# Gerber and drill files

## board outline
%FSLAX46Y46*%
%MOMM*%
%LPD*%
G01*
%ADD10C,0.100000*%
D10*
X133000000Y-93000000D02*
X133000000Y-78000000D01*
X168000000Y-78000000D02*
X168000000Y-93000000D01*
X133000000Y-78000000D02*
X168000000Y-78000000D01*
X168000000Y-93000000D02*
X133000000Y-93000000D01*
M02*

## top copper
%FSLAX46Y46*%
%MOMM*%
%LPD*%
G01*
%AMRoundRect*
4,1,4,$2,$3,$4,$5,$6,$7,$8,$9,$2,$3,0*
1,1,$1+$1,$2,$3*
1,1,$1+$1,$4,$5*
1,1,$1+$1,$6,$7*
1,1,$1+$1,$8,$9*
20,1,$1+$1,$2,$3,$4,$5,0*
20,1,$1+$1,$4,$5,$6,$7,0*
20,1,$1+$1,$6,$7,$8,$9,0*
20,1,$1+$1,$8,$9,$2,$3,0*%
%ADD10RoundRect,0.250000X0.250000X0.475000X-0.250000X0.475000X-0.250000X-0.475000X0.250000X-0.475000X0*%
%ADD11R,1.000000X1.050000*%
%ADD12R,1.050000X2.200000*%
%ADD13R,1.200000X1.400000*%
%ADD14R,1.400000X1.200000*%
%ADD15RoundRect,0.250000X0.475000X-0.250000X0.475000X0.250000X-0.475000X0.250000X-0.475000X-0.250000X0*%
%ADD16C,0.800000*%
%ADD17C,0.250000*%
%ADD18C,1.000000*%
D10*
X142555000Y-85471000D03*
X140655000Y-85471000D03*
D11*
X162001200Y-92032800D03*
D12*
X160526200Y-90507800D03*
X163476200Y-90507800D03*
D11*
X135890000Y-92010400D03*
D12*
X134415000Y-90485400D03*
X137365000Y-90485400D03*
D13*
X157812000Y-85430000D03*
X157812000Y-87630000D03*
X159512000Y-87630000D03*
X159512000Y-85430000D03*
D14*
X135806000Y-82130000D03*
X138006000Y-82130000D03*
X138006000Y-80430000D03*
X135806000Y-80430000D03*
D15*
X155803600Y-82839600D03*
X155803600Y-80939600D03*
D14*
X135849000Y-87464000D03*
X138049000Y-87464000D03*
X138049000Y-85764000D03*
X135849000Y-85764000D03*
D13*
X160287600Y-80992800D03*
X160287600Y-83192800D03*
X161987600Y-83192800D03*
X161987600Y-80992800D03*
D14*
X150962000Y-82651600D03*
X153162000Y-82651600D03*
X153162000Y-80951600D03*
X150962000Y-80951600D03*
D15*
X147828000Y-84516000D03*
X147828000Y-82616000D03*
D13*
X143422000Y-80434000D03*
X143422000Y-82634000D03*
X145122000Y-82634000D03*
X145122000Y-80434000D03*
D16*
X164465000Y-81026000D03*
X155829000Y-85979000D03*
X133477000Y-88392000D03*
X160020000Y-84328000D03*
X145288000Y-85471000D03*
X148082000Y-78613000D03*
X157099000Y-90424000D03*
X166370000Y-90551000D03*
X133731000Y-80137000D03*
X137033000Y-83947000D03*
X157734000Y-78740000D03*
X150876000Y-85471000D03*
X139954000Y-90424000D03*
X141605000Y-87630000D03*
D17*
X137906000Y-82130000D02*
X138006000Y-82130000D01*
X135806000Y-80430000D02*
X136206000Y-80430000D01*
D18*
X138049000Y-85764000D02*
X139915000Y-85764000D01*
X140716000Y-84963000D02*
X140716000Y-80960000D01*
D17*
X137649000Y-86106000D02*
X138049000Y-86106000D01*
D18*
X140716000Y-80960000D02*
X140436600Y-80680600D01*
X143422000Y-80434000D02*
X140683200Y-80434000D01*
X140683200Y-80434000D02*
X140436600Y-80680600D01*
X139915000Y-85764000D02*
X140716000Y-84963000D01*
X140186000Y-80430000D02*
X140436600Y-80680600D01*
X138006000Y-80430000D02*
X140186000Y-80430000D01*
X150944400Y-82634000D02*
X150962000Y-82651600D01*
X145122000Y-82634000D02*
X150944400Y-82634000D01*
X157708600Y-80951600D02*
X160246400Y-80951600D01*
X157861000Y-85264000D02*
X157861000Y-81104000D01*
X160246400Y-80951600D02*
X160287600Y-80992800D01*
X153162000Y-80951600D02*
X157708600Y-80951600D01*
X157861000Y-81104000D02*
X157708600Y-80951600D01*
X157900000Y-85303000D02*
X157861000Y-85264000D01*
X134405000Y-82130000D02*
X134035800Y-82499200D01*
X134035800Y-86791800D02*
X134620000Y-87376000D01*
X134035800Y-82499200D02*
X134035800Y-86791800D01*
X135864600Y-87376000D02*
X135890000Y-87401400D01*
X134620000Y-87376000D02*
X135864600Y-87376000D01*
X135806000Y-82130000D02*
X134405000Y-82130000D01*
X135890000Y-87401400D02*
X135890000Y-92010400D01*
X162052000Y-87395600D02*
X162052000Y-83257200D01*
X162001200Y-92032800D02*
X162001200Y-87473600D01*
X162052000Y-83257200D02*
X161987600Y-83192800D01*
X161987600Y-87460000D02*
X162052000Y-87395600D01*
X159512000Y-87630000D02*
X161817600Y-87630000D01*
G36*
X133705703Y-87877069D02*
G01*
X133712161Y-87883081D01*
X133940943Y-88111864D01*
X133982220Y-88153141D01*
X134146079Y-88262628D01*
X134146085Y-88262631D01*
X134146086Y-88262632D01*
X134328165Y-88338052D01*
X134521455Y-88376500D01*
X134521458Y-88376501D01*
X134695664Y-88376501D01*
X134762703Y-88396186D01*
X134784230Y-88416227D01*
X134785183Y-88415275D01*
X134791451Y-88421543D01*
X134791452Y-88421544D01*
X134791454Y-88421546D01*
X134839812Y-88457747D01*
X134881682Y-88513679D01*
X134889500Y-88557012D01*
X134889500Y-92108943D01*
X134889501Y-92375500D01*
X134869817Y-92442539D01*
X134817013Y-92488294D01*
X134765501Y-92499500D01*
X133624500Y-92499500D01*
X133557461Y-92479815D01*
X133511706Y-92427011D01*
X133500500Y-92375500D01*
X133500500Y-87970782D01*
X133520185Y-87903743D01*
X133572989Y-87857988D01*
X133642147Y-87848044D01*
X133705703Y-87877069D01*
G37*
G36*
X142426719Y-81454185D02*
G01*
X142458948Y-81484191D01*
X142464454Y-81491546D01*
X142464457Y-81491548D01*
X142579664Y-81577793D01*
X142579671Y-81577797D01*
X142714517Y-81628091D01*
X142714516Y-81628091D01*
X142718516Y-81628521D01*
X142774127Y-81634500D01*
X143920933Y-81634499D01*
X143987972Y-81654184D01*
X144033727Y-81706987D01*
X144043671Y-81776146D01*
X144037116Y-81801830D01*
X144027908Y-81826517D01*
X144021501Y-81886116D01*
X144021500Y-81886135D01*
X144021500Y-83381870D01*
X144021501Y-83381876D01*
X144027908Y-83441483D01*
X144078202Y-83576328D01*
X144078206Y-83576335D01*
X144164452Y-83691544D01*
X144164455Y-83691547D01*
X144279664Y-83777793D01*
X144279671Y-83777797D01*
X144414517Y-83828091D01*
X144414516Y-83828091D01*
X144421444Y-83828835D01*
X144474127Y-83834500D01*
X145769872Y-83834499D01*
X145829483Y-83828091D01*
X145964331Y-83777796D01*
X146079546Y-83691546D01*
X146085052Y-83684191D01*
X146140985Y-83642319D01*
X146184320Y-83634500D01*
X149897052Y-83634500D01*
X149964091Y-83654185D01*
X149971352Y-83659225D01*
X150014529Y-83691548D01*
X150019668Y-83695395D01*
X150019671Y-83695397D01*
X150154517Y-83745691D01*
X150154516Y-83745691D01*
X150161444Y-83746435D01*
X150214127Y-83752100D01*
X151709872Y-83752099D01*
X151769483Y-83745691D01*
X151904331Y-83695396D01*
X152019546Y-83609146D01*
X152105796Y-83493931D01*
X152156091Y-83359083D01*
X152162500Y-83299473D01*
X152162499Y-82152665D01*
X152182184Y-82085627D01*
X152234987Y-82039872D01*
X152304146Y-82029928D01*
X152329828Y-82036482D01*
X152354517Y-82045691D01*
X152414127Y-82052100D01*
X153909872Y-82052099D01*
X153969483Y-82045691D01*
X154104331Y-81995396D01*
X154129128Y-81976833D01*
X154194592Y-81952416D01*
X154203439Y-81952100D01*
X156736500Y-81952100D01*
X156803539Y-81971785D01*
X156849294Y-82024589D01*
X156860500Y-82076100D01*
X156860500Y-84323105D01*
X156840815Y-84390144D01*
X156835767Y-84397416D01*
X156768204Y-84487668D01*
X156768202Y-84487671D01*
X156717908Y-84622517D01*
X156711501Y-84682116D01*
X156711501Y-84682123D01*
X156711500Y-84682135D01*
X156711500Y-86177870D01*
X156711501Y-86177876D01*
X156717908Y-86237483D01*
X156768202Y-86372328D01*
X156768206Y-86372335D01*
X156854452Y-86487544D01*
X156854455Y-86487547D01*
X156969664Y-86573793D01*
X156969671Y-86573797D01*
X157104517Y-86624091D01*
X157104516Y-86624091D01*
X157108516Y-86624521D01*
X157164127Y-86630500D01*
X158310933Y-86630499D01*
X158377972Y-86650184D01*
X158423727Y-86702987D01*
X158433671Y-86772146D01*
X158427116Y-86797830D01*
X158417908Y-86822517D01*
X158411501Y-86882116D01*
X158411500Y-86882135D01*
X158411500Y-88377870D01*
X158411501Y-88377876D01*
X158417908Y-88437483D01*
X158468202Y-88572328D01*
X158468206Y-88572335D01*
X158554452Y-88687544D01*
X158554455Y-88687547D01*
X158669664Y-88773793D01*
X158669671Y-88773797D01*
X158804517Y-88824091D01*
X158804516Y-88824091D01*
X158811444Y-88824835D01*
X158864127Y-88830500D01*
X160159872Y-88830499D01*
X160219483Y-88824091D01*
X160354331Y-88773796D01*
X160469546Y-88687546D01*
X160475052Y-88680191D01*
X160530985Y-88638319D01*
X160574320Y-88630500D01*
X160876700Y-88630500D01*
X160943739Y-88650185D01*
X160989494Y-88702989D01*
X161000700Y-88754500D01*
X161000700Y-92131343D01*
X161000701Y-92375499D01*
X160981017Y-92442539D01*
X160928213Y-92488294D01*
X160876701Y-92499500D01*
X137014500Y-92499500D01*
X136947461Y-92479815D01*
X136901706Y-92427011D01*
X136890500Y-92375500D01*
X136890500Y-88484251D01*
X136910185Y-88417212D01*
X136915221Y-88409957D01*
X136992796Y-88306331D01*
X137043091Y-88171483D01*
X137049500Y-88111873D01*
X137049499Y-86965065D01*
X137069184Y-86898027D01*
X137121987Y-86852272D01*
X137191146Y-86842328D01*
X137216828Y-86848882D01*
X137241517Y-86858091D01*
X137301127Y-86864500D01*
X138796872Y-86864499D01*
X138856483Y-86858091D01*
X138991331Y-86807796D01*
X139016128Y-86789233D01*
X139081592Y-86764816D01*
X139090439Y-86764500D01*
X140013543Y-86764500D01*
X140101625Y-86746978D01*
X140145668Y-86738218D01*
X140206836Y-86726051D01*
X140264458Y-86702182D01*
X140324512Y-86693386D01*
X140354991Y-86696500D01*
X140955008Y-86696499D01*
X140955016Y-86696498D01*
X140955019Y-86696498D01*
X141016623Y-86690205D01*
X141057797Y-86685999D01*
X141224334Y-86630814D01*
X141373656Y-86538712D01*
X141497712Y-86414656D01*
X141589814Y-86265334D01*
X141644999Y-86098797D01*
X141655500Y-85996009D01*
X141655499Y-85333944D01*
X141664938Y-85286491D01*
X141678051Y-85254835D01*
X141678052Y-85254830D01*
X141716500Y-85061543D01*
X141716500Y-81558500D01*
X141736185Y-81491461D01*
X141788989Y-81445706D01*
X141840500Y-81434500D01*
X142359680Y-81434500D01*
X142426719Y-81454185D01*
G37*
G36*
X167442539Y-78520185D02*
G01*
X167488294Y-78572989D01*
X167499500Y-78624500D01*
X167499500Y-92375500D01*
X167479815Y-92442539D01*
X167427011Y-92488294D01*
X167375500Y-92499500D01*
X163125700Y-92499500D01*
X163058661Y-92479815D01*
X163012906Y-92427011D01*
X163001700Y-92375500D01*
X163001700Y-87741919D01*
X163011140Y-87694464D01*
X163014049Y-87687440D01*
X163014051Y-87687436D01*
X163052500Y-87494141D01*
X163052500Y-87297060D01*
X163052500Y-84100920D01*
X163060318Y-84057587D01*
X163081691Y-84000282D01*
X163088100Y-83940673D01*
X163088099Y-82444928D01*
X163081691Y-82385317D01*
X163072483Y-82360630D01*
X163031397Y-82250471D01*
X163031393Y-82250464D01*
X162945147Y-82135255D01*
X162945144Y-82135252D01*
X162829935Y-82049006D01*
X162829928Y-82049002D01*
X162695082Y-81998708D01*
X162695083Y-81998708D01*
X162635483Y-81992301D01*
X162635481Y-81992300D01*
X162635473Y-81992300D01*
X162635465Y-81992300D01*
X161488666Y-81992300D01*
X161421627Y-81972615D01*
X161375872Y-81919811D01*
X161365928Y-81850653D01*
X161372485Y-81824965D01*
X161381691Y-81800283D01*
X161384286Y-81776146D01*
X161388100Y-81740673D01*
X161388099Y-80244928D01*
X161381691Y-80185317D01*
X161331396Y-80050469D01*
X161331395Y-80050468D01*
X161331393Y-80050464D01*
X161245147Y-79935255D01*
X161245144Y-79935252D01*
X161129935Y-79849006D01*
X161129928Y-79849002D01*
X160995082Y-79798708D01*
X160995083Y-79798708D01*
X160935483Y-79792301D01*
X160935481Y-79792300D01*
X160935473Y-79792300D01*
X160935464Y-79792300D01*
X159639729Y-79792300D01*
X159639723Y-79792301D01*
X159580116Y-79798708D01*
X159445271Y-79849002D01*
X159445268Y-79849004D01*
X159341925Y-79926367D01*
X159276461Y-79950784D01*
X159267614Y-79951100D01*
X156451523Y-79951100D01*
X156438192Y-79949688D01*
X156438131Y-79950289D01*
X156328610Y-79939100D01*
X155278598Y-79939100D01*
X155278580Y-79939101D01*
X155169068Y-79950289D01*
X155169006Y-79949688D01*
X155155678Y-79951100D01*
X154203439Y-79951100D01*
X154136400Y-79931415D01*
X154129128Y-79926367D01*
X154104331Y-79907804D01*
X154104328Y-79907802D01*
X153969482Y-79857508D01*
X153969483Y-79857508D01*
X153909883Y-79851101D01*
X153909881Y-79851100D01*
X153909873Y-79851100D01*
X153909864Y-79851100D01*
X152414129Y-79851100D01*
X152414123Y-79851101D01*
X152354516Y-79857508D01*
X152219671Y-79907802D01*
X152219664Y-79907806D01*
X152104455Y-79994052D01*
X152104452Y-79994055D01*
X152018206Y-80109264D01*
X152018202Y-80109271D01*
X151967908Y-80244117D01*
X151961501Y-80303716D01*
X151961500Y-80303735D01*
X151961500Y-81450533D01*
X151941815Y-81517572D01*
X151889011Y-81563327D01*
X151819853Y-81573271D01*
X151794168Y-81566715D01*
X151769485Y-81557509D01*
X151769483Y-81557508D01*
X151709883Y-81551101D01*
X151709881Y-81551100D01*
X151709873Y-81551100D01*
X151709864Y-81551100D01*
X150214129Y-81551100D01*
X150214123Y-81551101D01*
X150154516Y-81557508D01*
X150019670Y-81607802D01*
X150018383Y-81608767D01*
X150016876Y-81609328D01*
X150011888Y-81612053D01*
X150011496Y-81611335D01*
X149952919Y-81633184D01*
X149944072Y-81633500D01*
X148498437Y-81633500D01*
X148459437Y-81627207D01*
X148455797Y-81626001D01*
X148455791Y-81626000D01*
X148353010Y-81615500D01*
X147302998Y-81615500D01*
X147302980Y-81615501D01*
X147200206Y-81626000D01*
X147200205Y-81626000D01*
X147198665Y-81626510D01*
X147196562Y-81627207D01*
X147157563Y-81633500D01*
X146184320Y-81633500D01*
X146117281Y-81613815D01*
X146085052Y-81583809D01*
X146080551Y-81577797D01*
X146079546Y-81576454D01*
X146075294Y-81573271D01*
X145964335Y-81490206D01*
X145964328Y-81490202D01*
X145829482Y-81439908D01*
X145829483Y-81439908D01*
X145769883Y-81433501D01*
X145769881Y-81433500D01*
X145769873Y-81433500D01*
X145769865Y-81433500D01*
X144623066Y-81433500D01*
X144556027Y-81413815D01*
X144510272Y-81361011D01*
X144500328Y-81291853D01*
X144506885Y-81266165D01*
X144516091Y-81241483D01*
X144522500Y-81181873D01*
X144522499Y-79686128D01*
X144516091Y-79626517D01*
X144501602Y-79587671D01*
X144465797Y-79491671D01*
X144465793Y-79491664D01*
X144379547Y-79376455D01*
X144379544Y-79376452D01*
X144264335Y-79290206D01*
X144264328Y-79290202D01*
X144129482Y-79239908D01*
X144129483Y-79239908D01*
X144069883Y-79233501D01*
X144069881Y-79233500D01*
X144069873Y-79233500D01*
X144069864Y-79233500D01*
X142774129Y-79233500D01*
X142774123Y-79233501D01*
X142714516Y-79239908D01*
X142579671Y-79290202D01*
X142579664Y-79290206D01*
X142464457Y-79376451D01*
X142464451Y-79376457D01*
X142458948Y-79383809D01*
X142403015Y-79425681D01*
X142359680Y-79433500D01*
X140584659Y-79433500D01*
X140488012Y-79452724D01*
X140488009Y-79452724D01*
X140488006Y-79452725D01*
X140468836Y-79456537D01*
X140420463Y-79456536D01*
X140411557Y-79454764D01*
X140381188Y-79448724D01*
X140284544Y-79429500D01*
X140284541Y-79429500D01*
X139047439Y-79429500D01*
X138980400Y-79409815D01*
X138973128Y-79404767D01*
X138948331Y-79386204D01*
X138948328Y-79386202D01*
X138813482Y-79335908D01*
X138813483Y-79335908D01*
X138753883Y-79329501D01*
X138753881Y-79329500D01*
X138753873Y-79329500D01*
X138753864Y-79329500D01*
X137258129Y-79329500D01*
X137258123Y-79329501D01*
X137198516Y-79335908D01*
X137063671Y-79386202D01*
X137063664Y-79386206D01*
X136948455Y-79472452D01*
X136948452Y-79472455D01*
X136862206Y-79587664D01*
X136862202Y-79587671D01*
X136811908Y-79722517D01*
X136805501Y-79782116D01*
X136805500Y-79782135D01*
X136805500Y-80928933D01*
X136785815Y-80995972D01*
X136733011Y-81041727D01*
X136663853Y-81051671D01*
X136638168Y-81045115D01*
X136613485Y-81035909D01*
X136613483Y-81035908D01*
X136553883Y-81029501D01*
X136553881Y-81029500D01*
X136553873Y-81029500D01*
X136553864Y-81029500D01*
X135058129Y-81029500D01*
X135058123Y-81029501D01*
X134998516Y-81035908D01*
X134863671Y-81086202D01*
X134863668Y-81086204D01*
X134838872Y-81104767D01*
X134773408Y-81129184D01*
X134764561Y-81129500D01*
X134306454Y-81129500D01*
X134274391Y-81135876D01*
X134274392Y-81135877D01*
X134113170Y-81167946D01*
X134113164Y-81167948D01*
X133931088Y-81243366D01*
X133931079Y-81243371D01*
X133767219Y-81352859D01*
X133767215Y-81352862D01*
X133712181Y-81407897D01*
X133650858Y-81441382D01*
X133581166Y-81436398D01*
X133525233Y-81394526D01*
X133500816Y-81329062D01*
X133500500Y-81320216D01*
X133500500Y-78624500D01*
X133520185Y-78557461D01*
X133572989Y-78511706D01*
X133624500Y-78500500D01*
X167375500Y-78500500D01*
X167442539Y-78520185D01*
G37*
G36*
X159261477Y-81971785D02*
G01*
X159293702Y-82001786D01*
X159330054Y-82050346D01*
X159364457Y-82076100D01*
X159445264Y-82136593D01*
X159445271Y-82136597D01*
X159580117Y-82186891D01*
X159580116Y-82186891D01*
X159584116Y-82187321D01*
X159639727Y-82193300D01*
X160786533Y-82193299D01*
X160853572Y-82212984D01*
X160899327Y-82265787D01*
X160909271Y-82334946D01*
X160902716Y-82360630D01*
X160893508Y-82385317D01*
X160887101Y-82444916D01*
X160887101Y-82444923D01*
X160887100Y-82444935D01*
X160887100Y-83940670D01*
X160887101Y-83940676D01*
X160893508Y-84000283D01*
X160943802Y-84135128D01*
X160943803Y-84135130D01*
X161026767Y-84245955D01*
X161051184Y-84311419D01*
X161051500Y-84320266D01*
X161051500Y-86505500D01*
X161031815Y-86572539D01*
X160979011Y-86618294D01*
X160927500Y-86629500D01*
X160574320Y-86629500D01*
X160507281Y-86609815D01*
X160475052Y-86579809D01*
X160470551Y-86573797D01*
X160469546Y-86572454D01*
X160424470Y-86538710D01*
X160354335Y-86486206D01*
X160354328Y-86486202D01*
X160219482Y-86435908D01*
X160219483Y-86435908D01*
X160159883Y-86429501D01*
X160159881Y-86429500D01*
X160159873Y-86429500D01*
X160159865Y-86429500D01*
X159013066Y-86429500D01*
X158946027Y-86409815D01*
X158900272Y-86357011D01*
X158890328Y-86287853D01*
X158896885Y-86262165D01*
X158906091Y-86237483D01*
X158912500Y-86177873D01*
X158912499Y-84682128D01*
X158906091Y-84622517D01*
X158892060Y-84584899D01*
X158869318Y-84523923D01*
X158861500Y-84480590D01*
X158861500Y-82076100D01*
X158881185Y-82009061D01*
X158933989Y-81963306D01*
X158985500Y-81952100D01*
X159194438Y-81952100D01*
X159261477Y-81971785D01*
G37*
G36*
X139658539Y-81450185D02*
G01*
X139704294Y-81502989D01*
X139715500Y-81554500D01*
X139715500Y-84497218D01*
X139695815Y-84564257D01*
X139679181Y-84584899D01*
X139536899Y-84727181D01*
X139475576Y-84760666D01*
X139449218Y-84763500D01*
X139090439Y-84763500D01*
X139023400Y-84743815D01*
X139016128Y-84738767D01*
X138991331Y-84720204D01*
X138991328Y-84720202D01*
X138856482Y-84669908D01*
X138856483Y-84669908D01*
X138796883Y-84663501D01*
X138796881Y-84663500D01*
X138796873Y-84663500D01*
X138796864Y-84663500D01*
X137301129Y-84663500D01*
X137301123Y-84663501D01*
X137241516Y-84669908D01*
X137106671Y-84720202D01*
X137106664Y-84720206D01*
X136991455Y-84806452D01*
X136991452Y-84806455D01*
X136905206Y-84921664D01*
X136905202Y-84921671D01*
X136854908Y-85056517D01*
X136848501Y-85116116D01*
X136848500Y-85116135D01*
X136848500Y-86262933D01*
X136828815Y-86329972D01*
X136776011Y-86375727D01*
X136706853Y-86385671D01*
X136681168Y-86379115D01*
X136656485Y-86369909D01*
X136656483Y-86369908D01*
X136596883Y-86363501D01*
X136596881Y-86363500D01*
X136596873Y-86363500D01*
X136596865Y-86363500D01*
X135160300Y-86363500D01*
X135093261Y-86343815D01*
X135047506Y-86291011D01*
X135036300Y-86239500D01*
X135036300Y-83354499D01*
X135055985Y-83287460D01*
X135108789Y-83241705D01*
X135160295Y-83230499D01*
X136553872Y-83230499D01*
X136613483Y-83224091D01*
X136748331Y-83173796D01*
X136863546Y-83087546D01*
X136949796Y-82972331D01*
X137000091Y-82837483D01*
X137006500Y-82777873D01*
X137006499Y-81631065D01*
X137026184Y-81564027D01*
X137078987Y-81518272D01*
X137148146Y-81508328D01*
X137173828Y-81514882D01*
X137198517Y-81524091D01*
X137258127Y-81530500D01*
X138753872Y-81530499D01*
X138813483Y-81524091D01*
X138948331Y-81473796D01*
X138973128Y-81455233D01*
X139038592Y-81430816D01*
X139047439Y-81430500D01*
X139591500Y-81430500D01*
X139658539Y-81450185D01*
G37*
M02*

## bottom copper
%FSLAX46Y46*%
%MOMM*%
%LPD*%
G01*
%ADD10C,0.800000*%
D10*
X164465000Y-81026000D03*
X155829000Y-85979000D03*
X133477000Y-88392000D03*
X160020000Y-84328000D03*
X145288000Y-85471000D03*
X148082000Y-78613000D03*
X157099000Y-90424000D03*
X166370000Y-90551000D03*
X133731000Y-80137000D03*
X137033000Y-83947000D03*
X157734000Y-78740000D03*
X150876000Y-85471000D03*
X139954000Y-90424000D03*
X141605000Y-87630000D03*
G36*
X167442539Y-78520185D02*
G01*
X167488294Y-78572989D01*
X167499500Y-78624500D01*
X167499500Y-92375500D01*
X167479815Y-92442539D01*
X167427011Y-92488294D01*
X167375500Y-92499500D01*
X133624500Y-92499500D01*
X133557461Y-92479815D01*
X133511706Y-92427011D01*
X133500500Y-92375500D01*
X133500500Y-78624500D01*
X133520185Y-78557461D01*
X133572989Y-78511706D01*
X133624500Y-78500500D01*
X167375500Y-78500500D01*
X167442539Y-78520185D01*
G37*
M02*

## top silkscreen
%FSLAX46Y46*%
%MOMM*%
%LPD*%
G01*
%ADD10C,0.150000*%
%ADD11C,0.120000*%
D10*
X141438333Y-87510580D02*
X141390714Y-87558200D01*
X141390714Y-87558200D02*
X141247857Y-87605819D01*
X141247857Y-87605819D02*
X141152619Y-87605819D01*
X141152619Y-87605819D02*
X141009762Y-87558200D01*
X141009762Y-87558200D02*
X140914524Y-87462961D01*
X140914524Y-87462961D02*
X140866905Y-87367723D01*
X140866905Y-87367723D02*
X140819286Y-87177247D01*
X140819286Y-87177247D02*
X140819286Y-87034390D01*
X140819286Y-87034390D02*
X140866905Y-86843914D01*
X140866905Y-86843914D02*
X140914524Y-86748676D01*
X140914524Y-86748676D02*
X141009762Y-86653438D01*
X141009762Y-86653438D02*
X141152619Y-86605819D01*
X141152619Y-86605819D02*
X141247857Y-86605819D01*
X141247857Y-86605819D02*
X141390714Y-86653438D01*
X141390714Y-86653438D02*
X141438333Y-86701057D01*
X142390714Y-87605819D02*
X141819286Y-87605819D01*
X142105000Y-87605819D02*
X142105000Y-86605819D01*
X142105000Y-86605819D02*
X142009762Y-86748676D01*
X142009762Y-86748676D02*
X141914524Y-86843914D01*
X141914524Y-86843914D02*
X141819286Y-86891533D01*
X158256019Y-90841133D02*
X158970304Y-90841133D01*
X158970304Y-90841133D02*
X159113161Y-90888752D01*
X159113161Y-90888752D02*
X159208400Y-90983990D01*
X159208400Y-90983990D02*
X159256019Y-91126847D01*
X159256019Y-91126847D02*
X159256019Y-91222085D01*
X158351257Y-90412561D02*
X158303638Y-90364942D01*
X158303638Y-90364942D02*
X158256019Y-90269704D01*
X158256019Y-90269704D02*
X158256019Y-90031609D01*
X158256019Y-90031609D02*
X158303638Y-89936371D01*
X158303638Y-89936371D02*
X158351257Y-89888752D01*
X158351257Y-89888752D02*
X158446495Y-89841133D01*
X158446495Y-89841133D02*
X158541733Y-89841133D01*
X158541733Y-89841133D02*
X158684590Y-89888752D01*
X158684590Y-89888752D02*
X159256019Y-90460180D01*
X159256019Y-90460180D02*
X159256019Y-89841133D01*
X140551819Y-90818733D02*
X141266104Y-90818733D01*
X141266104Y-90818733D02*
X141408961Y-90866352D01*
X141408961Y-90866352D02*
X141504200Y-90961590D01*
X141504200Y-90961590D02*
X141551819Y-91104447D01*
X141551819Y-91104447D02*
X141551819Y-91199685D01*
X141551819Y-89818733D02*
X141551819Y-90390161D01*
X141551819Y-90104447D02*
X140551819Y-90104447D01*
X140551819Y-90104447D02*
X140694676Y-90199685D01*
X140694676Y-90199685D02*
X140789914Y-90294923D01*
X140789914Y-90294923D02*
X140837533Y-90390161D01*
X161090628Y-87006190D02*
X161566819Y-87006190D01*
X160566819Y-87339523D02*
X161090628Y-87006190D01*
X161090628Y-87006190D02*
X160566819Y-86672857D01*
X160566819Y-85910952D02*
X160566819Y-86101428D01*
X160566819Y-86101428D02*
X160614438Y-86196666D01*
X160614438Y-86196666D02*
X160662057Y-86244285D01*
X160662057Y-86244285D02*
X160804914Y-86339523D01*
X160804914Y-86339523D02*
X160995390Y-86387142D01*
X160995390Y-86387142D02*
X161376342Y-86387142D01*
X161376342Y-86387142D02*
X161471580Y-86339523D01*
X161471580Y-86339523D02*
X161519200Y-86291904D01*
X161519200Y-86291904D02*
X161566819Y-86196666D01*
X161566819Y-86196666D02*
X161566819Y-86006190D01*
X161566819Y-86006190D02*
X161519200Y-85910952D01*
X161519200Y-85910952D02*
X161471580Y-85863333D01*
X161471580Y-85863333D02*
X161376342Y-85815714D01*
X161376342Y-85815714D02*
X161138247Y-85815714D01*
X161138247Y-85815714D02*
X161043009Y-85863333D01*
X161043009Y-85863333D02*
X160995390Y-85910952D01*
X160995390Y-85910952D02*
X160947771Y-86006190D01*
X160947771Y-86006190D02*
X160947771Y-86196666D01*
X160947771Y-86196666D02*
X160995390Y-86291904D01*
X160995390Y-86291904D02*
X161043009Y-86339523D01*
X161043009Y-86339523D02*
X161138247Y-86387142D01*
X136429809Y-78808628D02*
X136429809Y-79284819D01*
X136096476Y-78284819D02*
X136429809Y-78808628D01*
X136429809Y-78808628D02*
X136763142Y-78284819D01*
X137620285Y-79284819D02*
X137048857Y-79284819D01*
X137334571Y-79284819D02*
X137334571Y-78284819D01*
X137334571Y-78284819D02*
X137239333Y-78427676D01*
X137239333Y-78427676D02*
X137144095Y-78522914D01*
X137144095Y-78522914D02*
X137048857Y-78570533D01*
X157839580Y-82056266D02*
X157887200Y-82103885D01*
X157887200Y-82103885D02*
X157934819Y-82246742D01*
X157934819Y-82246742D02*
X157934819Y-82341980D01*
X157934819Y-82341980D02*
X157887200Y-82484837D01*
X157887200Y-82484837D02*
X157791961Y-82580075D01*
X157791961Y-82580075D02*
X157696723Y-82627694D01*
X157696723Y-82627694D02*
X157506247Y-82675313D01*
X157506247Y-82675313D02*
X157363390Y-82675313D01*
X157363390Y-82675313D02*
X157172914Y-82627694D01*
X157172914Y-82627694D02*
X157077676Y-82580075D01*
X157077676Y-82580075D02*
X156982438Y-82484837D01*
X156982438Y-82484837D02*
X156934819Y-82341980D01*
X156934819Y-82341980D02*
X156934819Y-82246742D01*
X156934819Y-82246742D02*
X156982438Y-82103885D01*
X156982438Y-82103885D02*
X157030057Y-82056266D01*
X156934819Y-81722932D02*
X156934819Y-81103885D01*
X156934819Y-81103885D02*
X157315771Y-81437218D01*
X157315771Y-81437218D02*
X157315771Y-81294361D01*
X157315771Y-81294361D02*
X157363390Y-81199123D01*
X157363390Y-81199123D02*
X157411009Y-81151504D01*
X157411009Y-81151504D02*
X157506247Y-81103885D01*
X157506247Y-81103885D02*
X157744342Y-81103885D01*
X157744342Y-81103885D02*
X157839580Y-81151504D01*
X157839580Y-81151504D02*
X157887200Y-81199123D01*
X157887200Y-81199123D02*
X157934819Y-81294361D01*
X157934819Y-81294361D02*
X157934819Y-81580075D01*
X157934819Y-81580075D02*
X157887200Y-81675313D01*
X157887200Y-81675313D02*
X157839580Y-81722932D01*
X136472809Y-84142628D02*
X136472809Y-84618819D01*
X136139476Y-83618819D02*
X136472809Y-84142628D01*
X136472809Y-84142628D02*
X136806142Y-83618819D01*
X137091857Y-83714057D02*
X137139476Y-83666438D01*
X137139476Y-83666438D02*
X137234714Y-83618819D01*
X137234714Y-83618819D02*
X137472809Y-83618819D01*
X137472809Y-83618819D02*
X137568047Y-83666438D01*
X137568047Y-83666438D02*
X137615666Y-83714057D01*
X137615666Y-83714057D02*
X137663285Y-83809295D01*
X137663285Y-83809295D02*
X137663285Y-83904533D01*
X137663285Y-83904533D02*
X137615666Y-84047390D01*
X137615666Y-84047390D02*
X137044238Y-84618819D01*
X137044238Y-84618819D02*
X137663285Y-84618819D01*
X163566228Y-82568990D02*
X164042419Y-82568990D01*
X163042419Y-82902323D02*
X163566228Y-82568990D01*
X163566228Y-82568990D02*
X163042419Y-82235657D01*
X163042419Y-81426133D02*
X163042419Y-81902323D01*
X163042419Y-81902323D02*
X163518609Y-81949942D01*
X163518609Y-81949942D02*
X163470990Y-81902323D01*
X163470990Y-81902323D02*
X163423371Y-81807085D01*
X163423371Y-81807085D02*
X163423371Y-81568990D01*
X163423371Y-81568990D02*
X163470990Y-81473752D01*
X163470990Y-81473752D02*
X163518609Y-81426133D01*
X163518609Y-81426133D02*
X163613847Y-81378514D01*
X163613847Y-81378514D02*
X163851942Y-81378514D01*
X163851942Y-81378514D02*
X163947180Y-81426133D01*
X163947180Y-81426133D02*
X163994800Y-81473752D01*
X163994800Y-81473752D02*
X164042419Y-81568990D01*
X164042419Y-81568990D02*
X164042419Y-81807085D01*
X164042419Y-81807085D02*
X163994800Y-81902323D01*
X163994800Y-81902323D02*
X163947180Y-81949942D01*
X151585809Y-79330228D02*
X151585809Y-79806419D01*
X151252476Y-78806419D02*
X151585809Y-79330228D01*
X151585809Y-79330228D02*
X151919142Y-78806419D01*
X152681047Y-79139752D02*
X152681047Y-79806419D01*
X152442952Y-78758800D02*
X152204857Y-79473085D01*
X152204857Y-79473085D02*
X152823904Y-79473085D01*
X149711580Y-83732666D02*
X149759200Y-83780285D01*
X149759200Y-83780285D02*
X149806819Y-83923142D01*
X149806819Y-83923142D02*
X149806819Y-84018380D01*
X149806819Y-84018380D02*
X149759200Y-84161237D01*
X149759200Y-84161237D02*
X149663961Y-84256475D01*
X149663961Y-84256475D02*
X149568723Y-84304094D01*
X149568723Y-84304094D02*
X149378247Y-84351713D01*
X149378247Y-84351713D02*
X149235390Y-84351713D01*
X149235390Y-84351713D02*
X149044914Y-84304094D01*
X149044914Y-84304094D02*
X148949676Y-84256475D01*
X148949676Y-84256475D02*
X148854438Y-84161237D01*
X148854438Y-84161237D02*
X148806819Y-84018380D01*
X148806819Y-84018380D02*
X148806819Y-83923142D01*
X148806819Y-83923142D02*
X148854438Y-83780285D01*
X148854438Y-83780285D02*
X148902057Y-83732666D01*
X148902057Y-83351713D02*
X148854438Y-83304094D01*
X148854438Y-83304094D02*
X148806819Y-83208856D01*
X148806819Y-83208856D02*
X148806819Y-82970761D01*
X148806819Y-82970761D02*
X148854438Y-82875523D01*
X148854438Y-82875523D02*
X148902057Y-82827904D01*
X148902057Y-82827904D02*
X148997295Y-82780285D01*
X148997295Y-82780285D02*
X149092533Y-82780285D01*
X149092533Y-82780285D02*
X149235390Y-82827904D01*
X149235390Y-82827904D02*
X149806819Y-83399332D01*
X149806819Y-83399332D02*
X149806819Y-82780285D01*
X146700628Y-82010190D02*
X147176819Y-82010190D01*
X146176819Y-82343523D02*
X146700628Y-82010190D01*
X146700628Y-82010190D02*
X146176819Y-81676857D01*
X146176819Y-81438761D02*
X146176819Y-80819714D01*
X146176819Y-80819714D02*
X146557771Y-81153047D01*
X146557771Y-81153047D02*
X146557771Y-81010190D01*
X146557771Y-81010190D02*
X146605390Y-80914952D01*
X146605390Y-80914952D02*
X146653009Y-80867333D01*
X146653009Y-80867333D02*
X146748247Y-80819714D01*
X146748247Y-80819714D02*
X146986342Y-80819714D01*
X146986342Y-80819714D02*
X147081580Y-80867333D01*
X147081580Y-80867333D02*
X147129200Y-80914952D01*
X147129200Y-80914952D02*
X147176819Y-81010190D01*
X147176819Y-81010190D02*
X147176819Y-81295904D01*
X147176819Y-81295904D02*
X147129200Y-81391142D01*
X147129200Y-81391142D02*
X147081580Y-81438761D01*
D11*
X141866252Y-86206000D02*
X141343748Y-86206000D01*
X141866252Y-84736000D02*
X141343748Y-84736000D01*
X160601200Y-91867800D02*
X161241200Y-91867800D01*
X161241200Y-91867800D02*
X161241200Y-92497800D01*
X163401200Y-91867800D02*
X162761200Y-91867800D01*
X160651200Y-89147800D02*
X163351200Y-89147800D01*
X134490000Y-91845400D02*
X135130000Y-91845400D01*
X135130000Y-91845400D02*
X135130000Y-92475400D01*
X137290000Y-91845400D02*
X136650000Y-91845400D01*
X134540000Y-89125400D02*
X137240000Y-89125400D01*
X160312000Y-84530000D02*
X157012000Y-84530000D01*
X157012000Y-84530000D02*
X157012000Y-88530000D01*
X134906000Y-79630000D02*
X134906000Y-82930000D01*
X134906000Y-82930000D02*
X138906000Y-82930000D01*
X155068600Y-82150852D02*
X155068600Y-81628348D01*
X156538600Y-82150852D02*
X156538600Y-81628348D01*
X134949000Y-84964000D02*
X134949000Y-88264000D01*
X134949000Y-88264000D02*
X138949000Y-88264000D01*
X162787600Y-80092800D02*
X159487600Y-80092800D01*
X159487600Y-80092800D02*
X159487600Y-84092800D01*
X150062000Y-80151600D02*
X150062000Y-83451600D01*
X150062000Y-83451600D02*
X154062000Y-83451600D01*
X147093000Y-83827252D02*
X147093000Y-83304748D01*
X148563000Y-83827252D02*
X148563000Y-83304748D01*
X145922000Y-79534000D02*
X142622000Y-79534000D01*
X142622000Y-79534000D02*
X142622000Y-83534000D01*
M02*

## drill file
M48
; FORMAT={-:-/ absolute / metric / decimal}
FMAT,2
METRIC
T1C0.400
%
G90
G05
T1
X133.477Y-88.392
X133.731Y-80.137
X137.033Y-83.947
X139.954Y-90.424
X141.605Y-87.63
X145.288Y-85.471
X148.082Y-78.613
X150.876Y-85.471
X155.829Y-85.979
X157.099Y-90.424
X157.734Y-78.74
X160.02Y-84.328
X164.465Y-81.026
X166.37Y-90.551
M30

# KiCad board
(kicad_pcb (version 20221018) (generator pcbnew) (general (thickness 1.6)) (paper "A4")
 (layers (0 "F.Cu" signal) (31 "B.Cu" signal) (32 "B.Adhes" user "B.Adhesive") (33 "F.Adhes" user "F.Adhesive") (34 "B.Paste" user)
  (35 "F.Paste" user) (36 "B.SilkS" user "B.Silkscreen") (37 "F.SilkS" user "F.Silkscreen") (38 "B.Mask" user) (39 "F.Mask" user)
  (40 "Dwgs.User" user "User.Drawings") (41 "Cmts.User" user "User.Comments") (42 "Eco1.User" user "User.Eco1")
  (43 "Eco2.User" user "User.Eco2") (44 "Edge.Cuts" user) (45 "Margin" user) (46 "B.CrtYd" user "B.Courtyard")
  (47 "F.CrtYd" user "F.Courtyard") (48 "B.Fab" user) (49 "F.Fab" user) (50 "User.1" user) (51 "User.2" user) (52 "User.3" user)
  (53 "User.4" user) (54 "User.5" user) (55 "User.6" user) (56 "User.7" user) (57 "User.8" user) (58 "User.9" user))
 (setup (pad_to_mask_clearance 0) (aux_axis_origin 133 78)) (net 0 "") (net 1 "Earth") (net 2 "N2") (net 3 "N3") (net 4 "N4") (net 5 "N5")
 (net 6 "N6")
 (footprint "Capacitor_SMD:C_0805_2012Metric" (layer "F.Cu") (at 141.605 85.471 180)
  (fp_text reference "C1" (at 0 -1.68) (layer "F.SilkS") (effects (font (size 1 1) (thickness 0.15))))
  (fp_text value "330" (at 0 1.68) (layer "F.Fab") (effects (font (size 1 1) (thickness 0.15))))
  (fp_line (start -0.261252 -0.735) (end 0.261252 -0.735) (stroke (width 0.12) (type solid)) (layer "F.SilkS"))
  (fp_line (start -0.261252 0.735) (end 0.261252 0.735) (stroke (width 0.12) (type solid)) (layer "F.SilkS"))
  (pad "1" smd roundrect (at -0.95 0 180) (size 1 1.45) (layers "F.Cu" "F.Paste" "F.Mask") (roundrect_rratio 0.25) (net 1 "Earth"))
  (pad "2" smd roundrect (at 0.95 0 180) (size 1 1.45) (layers "F.Cu" "F.Paste" "F.Mask") (roundrect_rratio 0.25) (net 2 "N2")))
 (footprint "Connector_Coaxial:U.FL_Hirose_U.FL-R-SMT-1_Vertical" (layer "F.Cu") (at 162.0012 90.9828 90)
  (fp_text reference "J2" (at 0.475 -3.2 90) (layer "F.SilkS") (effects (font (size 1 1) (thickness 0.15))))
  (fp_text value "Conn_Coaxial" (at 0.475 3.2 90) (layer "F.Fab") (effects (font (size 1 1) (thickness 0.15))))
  (fp_line (start -0.885 -1.4) (end -0.885 -0.76) (stroke (width 0.12) (type solid)) (layer "F.SilkS"))
  (fp_line (start -0.885 -0.76) (end -1.515 -0.76) (stroke (width 0.12) (type solid)) (layer "F.SilkS"))
  (fp_line (start -0.885 1.4) (end -0.885 0.76) (stroke (width 0.12) (type solid)) (layer "F.SilkS"))
  (fp_line (start 1.835 -1.35) (end 1.835 1.35) (stroke (width 0.12) (type solid)) (layer "F.SilkS"))
  (pad "1" smd rect (at -1.05 0 90) (size 1.05 1) (layers "F.Cu" "F.Paste" "F.Mask") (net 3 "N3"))
  (pad "2" smd rect (at 0.475 -1.475 90) (size 2.2 1.05) (layers "F.Cu" "F.Paste" "F.Mask") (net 1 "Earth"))
  (pad "2" smd rect (at 0.475 1.475 90) (size 2.2 1.05) (layers "F.Cu" "F.Paste" "F.Mask") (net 1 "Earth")))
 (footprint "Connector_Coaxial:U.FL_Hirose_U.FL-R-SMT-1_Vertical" (layer "F.Cu") (at 135.89 90.9604 90)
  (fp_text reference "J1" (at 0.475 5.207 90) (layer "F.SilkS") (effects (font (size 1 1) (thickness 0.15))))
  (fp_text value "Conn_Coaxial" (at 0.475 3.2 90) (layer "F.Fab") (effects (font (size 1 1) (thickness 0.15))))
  (fp_line (start -0.885 -1.4) (end -0.885 -0.76) (stroke (width 0.12) (type solid)) (layer "F.SilkS"))
  (fp_line (start -0.885 -0.76) (end -1.515 -0.76) (stroke (width 0.12) (type solid)) (layer "F.SilkS"))
  (fp_line (start -0.885 1.4) (end -0.885 0.76) (stroke (width 0.12) (type solid)) (layer "F.SilkS"))
  (fp_line (start 1.835 -1.35) (end 1.835 1.35) (stroke (width 0.12) (type solid)) (layer "F.SilkS"))
  (pad "1" smd rect (at -1.05 0 90) (size 1.05 1) (layers "F.Cu" "F.Paste" "F.Mask") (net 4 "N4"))
  (pad "2" smd rect (at 0.475 -1.475 90) (size 2.2 1.05) (layers "F.Cu" "F.Paste" "F.Mask") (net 1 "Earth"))
  (pad "2" smd rect (at 0.475 1.475 90) (size 2.2 1.05) (layers "F.Cu" "F.Paste" "F.Mask") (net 1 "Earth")))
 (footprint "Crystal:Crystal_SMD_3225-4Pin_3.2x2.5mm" (layer "F.Cu") (at 158.662 86.53 -90)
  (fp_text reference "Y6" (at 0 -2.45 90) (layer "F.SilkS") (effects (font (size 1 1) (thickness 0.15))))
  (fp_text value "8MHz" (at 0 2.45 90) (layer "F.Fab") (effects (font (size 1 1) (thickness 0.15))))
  (fp_line (start -2 -1.65) (end -2 1.65) (stroke (width 0.12) (type solid)) (layer "F.SilkS"))
  (fp_line (start -2 1.65) (end 2 1.65) (stroke (width 0.12) (type solid)) (layer "F.SilkS"))
  (pad "1" smd rect (at -1.1 0.85 270) (size 1.4 1.2) (layers "F.Cu" "F.Paste" "F.Mask") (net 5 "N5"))
  (pad "2" smd rect (at 1.1 0.85 270) (size 1.4 1.2) (layers "F.Cu" "F.Paste" "F.Mask") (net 1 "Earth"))
  (pad "3" smd rect (at 1.1 -0.85 270) (size 1.4 1.2) (layers "F.Cu" "F.Paste" "F.Mask") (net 3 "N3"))
  (pad "4" smd rect (at -1.1 -0.85 270) (size 1.4 1.2) (layers "F.Cu" "F.Paste" "F.Mask") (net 1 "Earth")))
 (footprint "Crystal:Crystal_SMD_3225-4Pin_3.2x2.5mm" (layer "F.Cu") (at 136.906 81.28)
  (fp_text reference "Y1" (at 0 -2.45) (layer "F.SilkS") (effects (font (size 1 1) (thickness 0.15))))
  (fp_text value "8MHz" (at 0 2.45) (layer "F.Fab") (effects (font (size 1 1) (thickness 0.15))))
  (fp_line (start -2 -1.65) (end -2 1.65) (stroke (width 0.12) (type solid)) (layer "F.SilkS"))
  (fp_line (start -2 1.65) (end 2 1.65) (stroke (width 0.12) (type solid)) (layer "F.SilkS"))
  (pad "1" smd rect (at -1.1 0.85) (size 1.4 1.2) (layers "F.Cu" "F.Paste" "F.Mask") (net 4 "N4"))
  (pad "2" smd rect (at 1.1 0.85) (size 1.4 1.2) (layers "F.Cu" "F.Paste" "F.Mask") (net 1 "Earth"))
  (pad "3" smd rect (at 1.1 -0.85) (size 1.4 1.2) (layers "F.Cu" "F.Paste" "F.Mask") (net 2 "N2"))
  (pad "4" smd rect (at -1.1 -0.85) (size 1.4 1.2) (layers "F.Cu" "F.Paste" "F.Mask") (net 1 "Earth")))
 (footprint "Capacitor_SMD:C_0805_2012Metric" (layer "F.Cu") (at 155.8036 81.8896 90)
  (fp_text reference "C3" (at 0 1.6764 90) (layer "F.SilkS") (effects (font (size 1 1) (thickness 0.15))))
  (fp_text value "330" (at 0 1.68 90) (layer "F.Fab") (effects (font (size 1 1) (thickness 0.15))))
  (fp_line (start -0.261252 -0.735) (end 0.261252 -0.735) (stroke (width 0.12) (type solid)) (layer "F.SilkS"))
  (fp_line (start -0.261252 0.735) (end 0.261252 0.735) (stroke (width 0.12) (type solid)) (layer "F.SilkS"))
  (pad "1" smd roundrect (at -0.95 0 90) (size 1 1.45) (layers "F.Cu" "F.Paste" "F.Mask") (roundrect_rratio 0.25) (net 1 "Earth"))
  (pad "2" smd roundrect (at 0.95 0 90) (size 1 1.45) (layers "F.Cu" "F.Paste" "F.Mask") (roundrect_rratio 0.25) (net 5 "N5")))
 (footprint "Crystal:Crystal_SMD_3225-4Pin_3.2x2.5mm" (layer "F.Cu") (at 136.949 86.614)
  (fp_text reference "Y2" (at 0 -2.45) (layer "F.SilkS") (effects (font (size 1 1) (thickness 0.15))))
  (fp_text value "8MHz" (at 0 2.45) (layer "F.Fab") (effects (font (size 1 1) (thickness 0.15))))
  (fp_line (start -2 -1.65) (end -2 1.65) (stroke (width 0.12) (type solid)) (layer "F.SilkS"))
  (fp_line (start -2 1.65) (end 2 1.65) (stroke (width 0.12) (type solid)) (layer "F.SilkS"))
  (pad "1" smd rect (at -1.1 0.85) (size 1.4 1.2) (layers "F.Cu" "F.Paste" "F.Mask") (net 4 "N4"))
  (pad "2" smd rect (at 1.1 0.85) (size 1.4 1.2) (layers "F.Cu" "F.Paste" "F.Mask") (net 1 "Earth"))
  (pad "3" smd rect (at 1.1 -0.85) (size 1.4 1.2) (layers "F.Cu" "F.Paste" "F.Mask") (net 2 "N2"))
  (pad "4" smd rect (at -1.1 -0.85) (size 1.4 1.2) (layers "F.Cu" "F.Paste" "F.Mask") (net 1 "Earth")))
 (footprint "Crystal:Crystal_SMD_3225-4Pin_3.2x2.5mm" (layer "F.Cu") (at 161.1376 82.0928 -90)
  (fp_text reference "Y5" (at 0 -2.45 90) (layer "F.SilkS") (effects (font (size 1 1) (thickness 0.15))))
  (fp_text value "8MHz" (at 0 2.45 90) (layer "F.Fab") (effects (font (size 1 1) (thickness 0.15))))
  (fp_line (start -2 -1.65) (end -2 1.65) (stroke (width 0.12) (type solid)) (layer "F.SilkS"))
  (fp_line (start -2 1.65) (end 2 1.65) (stroke (width 0.12) (type solid)) (layer "F.SilkS"))
  (pad "1" smd rect (at -1.1 0.85 270) (size 1.4 1.2) (layers "F.Cu" "F.Paste" "F.Mask") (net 5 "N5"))
  (pad "2" smd rect (at 1.1 0.85 270) (size 1.4 1.2) (layers "F.Cu" "F.Paste" "F.Mask") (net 1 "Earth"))
  (pad "3" smd rect (at 1.1 -0.85 270) (size 1.4 1.2) (layers "F.Cu" "F.Paste" "F.Mask") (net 3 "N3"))
  (pad "4" smd rect (at -1.1 -0.85 270) (size 1.4 1.2) (layers "F.Cu" "F.Paste" "F.Mask") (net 1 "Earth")))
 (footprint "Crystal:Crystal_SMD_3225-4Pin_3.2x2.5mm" (layer "F.Cu") (at 152.062 81.8016)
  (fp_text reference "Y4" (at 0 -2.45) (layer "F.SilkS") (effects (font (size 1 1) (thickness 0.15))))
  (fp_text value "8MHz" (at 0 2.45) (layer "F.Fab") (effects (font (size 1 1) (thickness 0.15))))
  (fp_line (start -2 -1.65) (end -2 1.65) (stroke (width 0.12) (type solid)) (layer "F.SilkS"))
  (fp_line (start -2 1.65) (end 2 1.65) (stroke (width 0.12) (type solid)) (layer "F.SilkS"))
  (pad "1" smd rect (at -1.1 0.85) (size 1.4 1.2) (layers "F.Cu" "F.Paste" "F.Mask") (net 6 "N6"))
  (pad "2" smd rect (at 1.1 0.85) (size 1.4 1.2) (layers "F.Cu" "F.Paste" "F.Mask") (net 1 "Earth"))
  (pad "3" smd rect (at 1.1 -0.85) (size 1.4 1.2) (layers "F.Cu" "F.Paste" "F.Mask") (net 5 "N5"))
  (pad "4" smd rect (at -1.1 -0.85) (size 1.4 1.2) (layers "F.Cu" "F.Paste" "F.Mask") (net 1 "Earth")))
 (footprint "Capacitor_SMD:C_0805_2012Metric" (layer "F.Cu") (at 147.828 83.566 90)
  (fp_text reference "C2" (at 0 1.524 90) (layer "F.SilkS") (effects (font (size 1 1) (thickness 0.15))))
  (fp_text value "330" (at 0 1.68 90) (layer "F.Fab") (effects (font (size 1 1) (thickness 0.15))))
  (fp_line (start -0.261252 -0.735) (end 0.261252 -0.735) (stroke (width 0.12) (type solid)) (layer "F.SilkS"))
  (fp_line (start -0.261252 0.735) (end 0.261252 0.735) (stroke (width 0.12) (type solid)) (layer "F.SilkS"))
  (pad "1" smd roundrect (at -0.95 0 90) (size 1 1.45) (layers "F.Cu" "F.Paste" "F.Mask") (roundrect_rratio 0.25) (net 1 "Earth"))
  (pad "2" smd roundrect (at 0.95 0 90) (size 1 1.45) (layers "F.Cu" "F.Paste" "F.Mask") (roundrect_rratio 0.25) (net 6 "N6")))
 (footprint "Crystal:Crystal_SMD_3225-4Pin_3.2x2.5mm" (layer "F.Cu") (at 144.272 81.534 -90)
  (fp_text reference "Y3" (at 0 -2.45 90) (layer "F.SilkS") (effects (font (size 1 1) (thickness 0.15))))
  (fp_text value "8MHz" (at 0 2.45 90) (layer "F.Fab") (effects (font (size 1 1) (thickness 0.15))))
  (fp_line (start -2 -1.65) (end -2 1.65) (stroke (width 0.12) (type solid)) (layer "F.SilkS"))
  (fp_line (start -2 1.65) (end 2 1.65) (stroke (width 0.12) (type solid)) (layer "F.SilkS"))
  (pad "1" smd rect (at -1.1 0.85 270) (size 1.4 1.2) (layers "F.Cu" "F.Paste" "F.Mask") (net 2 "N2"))
  (pad "2" smd rect (at 1.1 0.85 270) (size 1.4 1.2) (layers "F.Cu" "F.Paste" "F.Mask") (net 1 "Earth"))
  (pad "3" smd rect (at 1.1 -0.85 270) (size 1.4 1.2) (layers "F.Cu" "F.Paste" "F.Mask") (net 6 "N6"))
  (pad "4" smd rect (at -1.1 -0.85 270) (size 1.4 1.2) (layers "F.Cu" "F.Paste" "F.Mask") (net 1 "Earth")))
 (gr_line (start 133 93) (end 133 78) (stroke (width 0.1) (type default)) (layer "Edge.Cuts"))
 (gr_line (start 168 78) (end 168 93) (stroke (width 0.1) (type default)) (layer "Edge.Cuts"))
 (gr_line (start 133 78) (end 168 78) (stroke (width 0.1) (type default)) (layer "Edge.Cuts"))
 (gr_line (start 168 93) (end 133 93) (stroke (width 0.1) (type default)) (layer "Edge.Cuts"))
 (segment (start 137.906 82.13) (end 138.006 82.13) (width 0.25) (layer "F.Cu") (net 1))
 (segment (start 135.806 80.43) (end 136.206 80.43) (width 0.25) (layer "F.Cu") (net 1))
 (via (at 164.465 81.026) (size 0.8) (drill 0.4) (layers "F.Cu" "B.Cu") (free) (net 1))
 (via (at 155.829 85.979) (size 0.8) (drill 0.4) (layers "F.Cu" "B.Cu") (free) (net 1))
 (via (at 133.477 88.392) (size 0.8) (drill 0.4) (layers "F.Cu" "B.Cu") (free) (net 1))
 (via (at 160.02 84.328) (size 0.8) (drill 0.4) (layers "F.Cu" "B.Cu") (free) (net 1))
 (via (at 145.288 85.471) (size 0.8) (drill 0.4) (layers "F.Cu" "B.Cu") (free) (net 1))
 (via (at 148.082 78.613) (size 0.8) (drill 0.4) (layers "F.Cu" "B.Cu") (free) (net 1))
 (via (at 157.099 90.424) (size 0.8) (drill 0.4) (layers "F.Cu" "B.Cu") (free) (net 1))
 (via (at 166.37 90.551) (size 0.8) (drill 0.4) (layers "F.Cu" "B.Cu") (free) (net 1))
 (via (at 133.731 80.137) (size 0.8) (drill 0.4) (layers "F.Cu" "B.Cu") (free) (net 1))
 (via (at 137.033 83.947) (size 0.8) (drill 0.4) (layers "F.Cu" "B.Cu") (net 1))
 (via (at 157.734 78.74) (size 0.8) (drill 0.4) (layers "F.Cu" "B.Cu") (free) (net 1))
 (via (at 150.876 85.471) (size 0.8) (drill 0.4) (layers "F.Cu" "B.Cu") (free) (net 1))
 (via (at 139.954 90.424) (size 0.8) (drill 0.4) (layers "F.Cu" "B.Cu") (free) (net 1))
 (via (at 141.605 87.63) (size 0.8) (drill 0.4) (layers "F.Cu" "B.Cu") (free) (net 1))
 (segment (start 138.049 85.764) (end 139.915 85.764) (width 1) (layer "F.Cu") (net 2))
 (segment (start 140.716 84.963) (end 140.716 80.96) (width 1) (layer "F.Cu") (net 2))
 (segment (start 137.649 86.106) (end 138.049 86.106) (width 0.25) (layer "F.Cu") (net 2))
 (segment (start 140.716 80.96) (end 140.4366 80.6806) (width 1) (layer "F.Cu") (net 2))
 (segment (start 143.422 80.434) (end 140.6832 80.434) (width 1) (layer "F.Cu") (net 2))
 (segment (start 140.6832 80.434) (end 140.4366 80.6806) (width 1) (layer "F.Cu") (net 2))
 (segment (start 139.915 85.764) (end 140.716 84.963) (width 1) (layer "F.Cu") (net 2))
 (segment (start 140.186 80.43) (end 140.4366 80.6806) (width 1) (layer "F.Cu") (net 2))
 (segment (start 138.006 80.43) (end 140.186 80.43) (width 1) (layer "F.Cu") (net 2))
 (segment (start 150.9444 82.634) (end 150.962 82.6516) (width 1) (layer "F.Cu") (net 6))
 (segment (start 145.122 82.634) (end 150.9444 82.634) (width 1) (layer "F.Cu") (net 6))
 (segment (start 157.7086 80.9516) (end 160.2464 80.9516) (width 1) (layer "F.Cu") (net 5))
 (segment (start 157.861 85.264) (end 157.861 81.104) (width 1) (layer "F.Cu") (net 5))
 (segment (start 160.2464 80.9516) (end 160.2876 80.9928) (width 1) (layer "F.Cu") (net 5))
 (segment (start 153.162 80.9516) (end 157.7086 80.9516) (width 1) (layer "F.Cu") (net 5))
 (segment (start 157.861 81.104) (end 157.7086 80.9516) (width 1) (layer "F.Cu") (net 5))
 (segment (start 157.9 85.303) (end 157.861 85.264) (width 1) (layer "F.Cu") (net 5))
 (segment (start 134.405 82.13) (end 134.0358 82.4992) (width 1) (layer "F.Cu") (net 4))
 (segment (start 134.0358 86.7918) (end 134.62 87.376) (width 1) (layer "F.Cu") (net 4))
 (segment (start 134.0358 82.4992) (end 134.0358 86.7918) (width 1) (layer "F.Cu") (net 4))
 (segment (start 135.8646 87.376) (end 135.89 87.4014) (width 1) (layer "F.Cu") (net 4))
 (segment (start 134.62 87.376) (end 135.8646 87.376) (width 1) (layer "F.Cu") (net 4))
 (segment (start 135.806 82.13) (end 134.405 82.13) (width 1) (layer "F.Cu") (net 4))
 (segment (start 135.89 87.4014) (end 135.89 92.0104) (width 1) (layer "F.Cu") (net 4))
 (segment (start 162.052 87.3956) (end 162.052 83.2572) (width 1) (layer "F.Cu") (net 3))
 (segment (start 162.0012 92.0328) (end 162.0012 87.4736) (width 1) (layer "F.Cu") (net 3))
 (segment (start 162.052 83.2572) (end 161.9876 83.1928) (width 1) (layer "F.Cu") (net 3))
 (segment (start 161.9876 87.46) (end 162.052 87.3956) (width 1) (layer "F.Cu") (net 3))
 (segment (start 159.512 87.63) (end 161.8176 87.63) (width 1) (layer "F.Cu") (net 3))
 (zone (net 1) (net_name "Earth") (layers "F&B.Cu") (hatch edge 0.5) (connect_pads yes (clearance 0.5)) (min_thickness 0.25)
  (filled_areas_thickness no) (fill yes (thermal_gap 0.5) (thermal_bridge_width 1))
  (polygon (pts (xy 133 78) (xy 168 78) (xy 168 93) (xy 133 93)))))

